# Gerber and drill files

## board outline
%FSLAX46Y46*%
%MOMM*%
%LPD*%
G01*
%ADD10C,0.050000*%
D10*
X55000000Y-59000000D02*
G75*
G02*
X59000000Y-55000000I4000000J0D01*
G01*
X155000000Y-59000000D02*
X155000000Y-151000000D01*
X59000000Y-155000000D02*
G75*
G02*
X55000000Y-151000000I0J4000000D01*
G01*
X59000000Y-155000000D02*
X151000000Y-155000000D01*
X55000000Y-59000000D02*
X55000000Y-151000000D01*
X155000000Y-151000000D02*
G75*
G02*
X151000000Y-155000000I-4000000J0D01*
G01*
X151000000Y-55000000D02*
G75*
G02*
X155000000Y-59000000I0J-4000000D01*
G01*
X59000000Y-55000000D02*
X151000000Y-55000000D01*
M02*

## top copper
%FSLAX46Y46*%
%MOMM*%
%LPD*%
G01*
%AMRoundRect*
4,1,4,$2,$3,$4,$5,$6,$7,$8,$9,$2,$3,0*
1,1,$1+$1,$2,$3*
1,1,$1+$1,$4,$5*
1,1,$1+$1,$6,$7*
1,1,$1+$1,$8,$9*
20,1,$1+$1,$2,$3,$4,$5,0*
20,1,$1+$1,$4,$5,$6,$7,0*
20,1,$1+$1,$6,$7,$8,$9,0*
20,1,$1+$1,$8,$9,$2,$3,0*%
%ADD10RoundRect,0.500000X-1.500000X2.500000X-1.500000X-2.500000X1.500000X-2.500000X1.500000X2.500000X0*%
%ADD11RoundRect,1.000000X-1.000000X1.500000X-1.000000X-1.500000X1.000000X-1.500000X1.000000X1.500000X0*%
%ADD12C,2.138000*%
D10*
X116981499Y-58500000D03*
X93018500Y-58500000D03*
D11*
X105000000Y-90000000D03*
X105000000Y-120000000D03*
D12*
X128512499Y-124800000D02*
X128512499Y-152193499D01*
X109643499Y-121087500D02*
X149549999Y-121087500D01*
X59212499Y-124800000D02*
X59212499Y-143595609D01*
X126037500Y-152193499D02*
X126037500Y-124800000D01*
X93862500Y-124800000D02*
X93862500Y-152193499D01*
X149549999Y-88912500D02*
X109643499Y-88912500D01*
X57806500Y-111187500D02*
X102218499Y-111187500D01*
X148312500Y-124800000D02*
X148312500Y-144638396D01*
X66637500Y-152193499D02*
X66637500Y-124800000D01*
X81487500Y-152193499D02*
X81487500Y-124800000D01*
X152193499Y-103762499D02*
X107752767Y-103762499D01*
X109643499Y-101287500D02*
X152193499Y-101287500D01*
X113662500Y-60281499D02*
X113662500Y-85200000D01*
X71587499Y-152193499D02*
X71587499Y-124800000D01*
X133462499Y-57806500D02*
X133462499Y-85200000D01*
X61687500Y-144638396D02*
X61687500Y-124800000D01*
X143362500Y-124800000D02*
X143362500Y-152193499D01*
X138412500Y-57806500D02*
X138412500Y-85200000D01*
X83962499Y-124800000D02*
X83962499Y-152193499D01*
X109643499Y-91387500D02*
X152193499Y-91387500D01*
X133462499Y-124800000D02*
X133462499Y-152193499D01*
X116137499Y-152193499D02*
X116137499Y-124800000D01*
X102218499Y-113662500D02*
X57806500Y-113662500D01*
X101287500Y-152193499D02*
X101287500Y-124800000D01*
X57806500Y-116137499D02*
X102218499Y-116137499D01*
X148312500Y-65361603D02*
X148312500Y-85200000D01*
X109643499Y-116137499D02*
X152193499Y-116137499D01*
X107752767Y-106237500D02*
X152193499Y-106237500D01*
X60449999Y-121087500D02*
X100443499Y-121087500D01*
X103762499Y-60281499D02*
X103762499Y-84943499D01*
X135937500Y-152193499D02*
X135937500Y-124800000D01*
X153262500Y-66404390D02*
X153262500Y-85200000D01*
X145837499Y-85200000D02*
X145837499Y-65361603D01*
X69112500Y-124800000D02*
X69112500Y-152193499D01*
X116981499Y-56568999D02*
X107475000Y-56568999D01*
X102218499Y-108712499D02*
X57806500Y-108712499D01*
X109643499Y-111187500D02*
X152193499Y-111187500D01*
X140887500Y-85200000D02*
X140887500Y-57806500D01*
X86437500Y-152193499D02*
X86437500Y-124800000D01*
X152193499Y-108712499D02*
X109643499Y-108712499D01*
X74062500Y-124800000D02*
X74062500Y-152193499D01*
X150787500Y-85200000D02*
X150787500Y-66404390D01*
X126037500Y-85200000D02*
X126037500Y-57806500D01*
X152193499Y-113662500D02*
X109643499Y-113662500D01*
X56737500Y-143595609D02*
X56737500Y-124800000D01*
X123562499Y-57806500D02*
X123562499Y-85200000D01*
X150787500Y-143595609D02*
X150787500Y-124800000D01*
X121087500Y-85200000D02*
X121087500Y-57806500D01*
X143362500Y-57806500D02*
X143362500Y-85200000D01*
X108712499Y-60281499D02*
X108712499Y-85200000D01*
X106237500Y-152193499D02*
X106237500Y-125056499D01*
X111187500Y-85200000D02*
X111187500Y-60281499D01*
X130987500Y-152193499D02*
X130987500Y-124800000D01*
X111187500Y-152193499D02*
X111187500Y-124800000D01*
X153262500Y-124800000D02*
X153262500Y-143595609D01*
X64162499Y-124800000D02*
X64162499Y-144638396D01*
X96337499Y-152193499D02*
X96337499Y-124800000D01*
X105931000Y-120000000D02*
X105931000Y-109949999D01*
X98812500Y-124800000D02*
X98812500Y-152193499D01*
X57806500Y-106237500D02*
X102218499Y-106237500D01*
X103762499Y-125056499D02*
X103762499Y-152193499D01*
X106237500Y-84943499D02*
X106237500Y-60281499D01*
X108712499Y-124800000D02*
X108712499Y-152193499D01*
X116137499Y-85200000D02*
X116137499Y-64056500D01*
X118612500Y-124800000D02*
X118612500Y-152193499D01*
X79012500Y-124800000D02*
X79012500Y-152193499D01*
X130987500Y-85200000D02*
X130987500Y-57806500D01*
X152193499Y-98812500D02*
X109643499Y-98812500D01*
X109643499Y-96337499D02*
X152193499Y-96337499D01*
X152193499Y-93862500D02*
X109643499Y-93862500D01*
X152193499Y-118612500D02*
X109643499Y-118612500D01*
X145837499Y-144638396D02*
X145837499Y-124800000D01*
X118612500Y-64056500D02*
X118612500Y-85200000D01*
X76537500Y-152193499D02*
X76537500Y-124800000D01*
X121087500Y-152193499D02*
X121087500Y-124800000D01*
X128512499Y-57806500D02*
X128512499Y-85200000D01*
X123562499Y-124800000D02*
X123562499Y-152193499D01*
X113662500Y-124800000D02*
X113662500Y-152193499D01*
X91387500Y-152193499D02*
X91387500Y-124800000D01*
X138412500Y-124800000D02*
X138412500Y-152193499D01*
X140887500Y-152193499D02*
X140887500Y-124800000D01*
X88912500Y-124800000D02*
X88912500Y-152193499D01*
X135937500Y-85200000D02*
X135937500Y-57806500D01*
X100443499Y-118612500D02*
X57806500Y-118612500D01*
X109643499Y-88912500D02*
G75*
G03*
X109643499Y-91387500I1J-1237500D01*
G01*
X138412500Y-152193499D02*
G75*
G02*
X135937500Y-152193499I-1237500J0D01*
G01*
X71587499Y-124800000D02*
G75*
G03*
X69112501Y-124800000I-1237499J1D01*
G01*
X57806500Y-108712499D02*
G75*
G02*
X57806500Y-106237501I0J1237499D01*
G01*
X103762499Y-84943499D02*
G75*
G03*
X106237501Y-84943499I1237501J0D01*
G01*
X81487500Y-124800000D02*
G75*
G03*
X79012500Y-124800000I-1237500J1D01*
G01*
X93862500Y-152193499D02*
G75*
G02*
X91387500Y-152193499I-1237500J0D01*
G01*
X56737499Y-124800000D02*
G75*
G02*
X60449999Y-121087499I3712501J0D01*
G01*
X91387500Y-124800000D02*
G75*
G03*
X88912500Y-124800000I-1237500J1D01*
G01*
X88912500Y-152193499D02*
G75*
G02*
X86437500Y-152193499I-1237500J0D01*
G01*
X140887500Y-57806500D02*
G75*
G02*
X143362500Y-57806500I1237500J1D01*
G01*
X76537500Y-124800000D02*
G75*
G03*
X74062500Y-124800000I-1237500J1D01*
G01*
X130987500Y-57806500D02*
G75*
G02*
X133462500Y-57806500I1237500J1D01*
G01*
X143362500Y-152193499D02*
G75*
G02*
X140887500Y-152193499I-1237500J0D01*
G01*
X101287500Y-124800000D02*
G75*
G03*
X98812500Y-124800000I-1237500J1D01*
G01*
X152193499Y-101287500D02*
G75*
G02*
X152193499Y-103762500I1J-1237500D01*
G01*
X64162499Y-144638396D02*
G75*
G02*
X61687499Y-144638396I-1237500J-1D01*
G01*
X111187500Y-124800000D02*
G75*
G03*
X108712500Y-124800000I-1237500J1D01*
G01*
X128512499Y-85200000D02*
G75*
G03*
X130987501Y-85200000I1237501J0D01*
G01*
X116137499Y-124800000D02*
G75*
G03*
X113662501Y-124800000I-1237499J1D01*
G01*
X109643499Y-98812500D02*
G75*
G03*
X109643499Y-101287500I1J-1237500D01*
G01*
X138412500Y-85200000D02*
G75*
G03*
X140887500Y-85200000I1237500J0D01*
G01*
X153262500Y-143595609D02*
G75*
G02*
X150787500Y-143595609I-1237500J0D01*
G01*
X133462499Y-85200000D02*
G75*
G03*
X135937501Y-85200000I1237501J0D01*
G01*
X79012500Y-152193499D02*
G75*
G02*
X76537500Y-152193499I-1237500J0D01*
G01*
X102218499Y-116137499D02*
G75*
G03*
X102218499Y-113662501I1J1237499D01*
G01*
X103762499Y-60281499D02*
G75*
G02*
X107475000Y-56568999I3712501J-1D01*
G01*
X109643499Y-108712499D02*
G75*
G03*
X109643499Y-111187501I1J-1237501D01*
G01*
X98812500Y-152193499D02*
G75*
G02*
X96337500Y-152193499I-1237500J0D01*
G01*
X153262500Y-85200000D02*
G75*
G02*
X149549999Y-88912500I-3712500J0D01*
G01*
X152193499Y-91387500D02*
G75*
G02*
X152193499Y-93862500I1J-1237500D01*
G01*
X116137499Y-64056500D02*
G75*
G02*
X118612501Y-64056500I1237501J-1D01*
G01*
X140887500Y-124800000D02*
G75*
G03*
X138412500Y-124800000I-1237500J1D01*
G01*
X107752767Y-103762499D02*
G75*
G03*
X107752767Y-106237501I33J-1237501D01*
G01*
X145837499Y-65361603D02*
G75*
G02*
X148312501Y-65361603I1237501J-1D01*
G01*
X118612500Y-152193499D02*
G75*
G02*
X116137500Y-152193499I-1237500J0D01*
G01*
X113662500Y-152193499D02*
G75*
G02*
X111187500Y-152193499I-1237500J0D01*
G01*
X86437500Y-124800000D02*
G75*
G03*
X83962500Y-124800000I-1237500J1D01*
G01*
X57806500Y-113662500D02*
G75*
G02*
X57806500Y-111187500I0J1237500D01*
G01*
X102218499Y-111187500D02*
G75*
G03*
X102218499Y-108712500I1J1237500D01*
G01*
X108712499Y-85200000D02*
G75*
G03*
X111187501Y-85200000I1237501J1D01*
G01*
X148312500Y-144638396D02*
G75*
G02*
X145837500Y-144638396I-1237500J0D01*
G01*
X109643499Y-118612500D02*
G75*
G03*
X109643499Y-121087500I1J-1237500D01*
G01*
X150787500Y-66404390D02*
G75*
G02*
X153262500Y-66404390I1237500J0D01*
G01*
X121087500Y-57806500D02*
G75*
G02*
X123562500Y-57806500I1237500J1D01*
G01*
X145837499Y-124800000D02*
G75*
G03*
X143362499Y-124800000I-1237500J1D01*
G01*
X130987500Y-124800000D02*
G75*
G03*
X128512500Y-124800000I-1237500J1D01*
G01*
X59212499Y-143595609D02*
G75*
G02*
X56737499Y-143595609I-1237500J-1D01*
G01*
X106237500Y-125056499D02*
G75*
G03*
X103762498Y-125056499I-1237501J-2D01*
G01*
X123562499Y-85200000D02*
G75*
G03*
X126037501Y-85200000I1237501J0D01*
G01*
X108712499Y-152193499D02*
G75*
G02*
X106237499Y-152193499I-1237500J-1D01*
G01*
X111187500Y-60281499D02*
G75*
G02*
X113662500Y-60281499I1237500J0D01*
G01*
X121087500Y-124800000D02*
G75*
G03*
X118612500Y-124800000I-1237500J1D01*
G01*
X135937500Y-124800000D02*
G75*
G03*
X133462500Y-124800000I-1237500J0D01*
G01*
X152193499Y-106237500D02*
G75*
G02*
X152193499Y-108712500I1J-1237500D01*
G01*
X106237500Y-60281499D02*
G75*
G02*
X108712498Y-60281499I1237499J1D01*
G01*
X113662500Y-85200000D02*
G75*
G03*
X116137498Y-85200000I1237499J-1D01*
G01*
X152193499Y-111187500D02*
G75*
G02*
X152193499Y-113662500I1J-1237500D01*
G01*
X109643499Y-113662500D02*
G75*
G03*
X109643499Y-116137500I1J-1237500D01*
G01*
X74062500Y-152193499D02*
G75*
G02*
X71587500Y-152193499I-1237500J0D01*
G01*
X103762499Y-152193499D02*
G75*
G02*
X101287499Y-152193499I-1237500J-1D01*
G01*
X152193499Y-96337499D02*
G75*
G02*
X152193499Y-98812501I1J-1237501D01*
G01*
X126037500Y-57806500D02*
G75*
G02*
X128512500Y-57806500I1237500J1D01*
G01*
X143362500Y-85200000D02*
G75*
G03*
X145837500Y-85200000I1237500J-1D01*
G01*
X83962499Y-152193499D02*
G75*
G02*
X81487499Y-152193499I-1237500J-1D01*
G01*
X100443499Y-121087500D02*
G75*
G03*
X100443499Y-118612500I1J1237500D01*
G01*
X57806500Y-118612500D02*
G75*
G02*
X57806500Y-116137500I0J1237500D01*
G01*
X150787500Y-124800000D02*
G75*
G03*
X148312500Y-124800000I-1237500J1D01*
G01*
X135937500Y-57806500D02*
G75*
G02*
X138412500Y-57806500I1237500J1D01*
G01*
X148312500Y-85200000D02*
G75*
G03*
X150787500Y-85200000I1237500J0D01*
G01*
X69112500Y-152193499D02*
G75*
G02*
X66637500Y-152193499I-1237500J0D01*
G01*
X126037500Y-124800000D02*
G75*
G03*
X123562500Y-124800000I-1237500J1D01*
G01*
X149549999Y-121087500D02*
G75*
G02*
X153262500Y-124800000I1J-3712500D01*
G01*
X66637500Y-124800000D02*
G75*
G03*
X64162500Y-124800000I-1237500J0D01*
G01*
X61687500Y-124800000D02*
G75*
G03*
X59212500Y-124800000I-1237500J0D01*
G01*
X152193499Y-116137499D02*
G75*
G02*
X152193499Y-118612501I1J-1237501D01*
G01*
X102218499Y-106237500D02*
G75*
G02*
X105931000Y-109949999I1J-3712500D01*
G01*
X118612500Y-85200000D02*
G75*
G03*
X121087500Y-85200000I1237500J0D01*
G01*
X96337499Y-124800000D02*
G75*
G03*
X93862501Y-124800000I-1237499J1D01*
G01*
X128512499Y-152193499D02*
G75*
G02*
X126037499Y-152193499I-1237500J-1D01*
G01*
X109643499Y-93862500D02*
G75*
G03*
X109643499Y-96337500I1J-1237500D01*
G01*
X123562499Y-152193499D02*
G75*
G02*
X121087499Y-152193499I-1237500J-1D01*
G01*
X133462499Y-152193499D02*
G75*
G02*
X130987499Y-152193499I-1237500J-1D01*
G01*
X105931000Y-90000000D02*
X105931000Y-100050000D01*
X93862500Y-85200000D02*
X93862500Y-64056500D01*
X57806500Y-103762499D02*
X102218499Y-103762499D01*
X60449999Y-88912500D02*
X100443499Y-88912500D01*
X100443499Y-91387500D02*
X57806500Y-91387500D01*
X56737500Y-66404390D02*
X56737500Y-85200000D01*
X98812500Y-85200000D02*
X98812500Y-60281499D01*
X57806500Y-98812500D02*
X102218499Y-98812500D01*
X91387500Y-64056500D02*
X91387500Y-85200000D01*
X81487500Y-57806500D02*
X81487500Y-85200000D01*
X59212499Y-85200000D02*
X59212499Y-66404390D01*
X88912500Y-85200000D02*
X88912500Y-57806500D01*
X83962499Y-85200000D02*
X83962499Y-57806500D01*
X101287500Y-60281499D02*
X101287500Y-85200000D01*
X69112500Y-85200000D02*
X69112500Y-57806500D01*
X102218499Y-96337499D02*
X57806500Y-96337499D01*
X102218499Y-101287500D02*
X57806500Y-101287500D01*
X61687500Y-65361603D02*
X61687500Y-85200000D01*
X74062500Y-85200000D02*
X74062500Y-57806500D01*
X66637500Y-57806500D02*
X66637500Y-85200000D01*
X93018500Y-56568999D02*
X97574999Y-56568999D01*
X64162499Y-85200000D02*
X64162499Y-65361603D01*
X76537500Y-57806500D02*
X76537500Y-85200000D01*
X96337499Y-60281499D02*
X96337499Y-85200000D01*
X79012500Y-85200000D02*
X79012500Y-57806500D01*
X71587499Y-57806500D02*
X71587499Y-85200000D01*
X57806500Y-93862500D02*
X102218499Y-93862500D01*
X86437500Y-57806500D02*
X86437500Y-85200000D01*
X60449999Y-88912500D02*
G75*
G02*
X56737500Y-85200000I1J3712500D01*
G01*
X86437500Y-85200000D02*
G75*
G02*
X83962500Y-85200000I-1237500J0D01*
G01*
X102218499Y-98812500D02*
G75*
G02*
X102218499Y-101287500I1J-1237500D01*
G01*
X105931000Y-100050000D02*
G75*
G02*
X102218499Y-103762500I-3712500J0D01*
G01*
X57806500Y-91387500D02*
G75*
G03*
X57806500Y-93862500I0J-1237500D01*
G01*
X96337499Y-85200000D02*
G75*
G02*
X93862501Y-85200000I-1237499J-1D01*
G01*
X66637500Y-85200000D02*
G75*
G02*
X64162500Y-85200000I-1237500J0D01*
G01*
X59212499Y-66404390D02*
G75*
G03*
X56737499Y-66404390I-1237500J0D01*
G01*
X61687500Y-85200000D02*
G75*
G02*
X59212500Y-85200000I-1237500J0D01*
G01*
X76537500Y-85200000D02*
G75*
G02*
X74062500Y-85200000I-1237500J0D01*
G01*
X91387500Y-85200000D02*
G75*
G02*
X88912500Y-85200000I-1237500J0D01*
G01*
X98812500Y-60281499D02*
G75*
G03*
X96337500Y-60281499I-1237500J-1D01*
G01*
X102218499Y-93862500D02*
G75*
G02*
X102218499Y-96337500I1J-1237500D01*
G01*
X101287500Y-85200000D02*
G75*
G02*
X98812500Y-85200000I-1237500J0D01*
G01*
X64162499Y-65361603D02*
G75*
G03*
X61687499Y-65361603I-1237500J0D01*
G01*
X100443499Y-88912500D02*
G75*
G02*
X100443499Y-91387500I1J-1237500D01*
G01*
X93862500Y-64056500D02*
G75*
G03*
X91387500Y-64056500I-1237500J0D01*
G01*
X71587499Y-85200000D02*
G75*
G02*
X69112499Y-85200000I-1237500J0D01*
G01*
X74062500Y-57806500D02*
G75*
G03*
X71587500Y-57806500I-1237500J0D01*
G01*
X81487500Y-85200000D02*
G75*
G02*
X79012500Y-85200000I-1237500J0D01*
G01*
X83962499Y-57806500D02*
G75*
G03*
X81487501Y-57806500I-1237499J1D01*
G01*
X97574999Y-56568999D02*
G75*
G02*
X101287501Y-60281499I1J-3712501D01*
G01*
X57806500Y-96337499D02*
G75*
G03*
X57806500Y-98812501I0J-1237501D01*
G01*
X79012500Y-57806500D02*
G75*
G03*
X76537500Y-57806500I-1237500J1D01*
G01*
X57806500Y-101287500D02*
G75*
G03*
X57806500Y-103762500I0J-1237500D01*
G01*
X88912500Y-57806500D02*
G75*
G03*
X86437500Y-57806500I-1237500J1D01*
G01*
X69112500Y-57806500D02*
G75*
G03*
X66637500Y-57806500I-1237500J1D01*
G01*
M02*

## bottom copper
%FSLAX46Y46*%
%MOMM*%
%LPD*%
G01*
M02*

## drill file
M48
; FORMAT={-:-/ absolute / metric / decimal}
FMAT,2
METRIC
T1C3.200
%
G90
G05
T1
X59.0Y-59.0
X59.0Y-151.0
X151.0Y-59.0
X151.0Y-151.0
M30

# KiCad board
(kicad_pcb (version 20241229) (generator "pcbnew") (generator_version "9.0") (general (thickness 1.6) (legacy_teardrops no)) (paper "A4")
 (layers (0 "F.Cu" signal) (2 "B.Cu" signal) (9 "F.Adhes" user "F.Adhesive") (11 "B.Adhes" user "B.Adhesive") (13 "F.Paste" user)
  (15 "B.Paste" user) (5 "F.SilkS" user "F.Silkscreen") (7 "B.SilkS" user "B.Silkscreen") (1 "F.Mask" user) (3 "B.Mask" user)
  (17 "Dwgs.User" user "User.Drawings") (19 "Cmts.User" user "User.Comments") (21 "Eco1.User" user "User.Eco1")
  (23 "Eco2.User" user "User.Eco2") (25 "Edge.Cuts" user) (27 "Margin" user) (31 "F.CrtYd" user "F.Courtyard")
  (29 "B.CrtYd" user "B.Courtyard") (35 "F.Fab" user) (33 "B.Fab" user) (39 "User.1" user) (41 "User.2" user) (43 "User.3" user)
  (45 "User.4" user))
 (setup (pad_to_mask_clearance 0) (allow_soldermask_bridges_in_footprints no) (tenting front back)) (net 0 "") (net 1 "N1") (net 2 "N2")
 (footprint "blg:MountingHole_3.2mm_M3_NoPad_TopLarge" (layer "F.Cu") (at 151 59)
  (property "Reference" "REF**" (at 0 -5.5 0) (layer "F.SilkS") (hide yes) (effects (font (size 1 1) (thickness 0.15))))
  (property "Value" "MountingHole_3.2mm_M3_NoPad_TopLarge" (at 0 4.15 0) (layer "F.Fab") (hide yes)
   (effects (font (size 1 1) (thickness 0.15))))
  (pad "" np_thru_hole circle (at 0 0) (size 7.6 7.6) (drill 3.2) (layers) (zone_connect 2)))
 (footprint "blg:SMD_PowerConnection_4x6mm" (layer "F.Cu") (at 116.981499 58.5 -90)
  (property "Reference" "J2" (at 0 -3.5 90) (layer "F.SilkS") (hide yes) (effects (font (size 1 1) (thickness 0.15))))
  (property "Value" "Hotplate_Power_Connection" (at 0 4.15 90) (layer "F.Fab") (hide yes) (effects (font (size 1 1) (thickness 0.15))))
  (pad "1" smd roundrect (at 0 0 270) (size 6 4) (layers "F.Cu" "F.Mask" "F.Paste") (roundrect_rratio 0.125) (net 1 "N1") (zone_connect 2)))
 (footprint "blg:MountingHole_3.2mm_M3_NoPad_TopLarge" (layer "F.Cu") (at 59 151)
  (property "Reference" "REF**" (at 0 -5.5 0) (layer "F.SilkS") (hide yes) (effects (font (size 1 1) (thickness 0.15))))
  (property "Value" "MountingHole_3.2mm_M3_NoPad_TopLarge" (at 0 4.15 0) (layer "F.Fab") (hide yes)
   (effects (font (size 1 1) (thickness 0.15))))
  (pad "" np_thru_hole circle (at 0 0) (size 7.6 7.6) (drill 3.2) (layers) (zone_connect 2)))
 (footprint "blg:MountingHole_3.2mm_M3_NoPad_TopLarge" (layer "F.Cu") (at 151 151)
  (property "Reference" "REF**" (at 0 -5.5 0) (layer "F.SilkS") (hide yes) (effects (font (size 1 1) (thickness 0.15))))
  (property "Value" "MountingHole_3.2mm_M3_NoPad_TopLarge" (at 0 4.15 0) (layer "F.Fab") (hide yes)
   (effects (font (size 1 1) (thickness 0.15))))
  (pad "" np_thru_hole circle (at 0 0) (size 7.6 7.6) (drill 3.2) (layers) (zone_connect 2)))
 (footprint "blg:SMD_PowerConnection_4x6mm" (layer "F.Cu") (at 93.0185 58.5 -90)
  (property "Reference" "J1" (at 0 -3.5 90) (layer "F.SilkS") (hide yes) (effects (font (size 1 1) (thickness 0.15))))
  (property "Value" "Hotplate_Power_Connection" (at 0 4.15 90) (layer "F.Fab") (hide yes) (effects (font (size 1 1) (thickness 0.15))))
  (pad "1" smd roundrect (at 0 0 270) (size 6 4) (layers "F.Cu" "F.Mask" "F.Paste") (roundrect_rratio 0.125) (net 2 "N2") (zone_connect 2)))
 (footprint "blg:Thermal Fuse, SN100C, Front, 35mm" (layer "F.Cu") (at 105 105 -90)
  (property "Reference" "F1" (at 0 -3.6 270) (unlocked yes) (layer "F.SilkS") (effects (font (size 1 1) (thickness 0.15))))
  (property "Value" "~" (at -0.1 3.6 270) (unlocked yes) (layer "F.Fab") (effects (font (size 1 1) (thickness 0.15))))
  (pad "1" smd roundrect (at -15 0 270) (size 5 4) (layers "F.Cu" "F.Mask") (roundrect_rratio 0.25) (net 2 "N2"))
  (pad "2" smd roundrect (at 15 0 270) (size 5 4) (layers "F.Cu" "F.Mask") (roundrect_rratio 0.25) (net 1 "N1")))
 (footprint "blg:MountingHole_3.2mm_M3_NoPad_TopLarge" (layer "F.Cu") (at 59 59)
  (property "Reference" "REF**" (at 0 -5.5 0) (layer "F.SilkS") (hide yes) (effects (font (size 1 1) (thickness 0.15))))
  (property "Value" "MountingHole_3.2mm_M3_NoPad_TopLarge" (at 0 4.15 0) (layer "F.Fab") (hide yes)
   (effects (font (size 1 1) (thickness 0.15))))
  (pad "" np_thru_hole circle (at 0 0) (size 7.6 7.6) (drill 3.2) (layers) (zone_connect 2)))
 (gr_arc (start 55 59) (mid 56.171573 56.171573) (end 59 55) (stroke (width 0.05) (type solid)) (layer "Edge.Cuts"))
 (gr_line (start 155 59) (end 155 151) (stroke (width 0.05) (type default)) (layer "Edge.Cuts"))
 (gr_arc (start 59 155) (mid 56.171573 153.828427) (end 55 151) (stroke (width 0.05) (type solid)) (layer "Edge.Cuts"))
 (gr_line (start 59 155) (end 151 155) (stroke (width 0.05) (type default)) (layer "Edge.Cuts"))
 (gr_line (start 55 59) (end 55 151) (stroke (width 0.05) (type default)) (layer "Edge.Cuts"))
 (gr_arc (start 155 151) (mid 153.828427 153.828427) (end 151 155) (stroke (width 0.05) (type solid)) (layer "Edge.Cuts"))
 (gr_arc (start 151 55) (mid 153.828427 56.171573) (end 155 59) (stroke (width 0.05) (type solid)) (layer "Edge.Cuts"))
 (gr_line (start 59 55) (end 151 55) (stroke (width 0.05) (type default)) (layer "Edge.Cuts"))
 (segment (start 128.512499 124.8) (end 128.512499 152.193499) (width 2.138) (layer "F.Cu") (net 1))
 (segment (start 109.643499 121.0875) (end 149.549999 121.0875) (width 2.138) (layer "F.Cu") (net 1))
 (segment (start 59.212499 124.8) (end 59.212499 143.595609) (width 2.138) (layer "F.Cu") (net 1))
 (segment (start 126.0375 152.193499) (end 126.0375 124.8) (width 2.138) (layer "F.Cu") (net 1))
 (segment (start 93.8625 124.8) (end 93.8625 152.193499) (width 2.138) (layer "F.Cu") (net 1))
 (segment (start 149.549999 88.9125) (end 109.643499 88.9125) (width 2.138) (layer "F.Cu") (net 1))
 (segment (start 57.8065 111.1875) (end 102.218499 111.1875) (width 2.138) (layer "F.Cu") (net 1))
 (segment (start 148.3125 124.8) (end 148.3125 144.638396) (width 2.138) (layer "F.Cu") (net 1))
 (segment (start 66.6375 152.193499) (end 66.6375 124.8) (width 2.138) (layer "F.Cu") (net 1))
 (segment (start 81.4875 152.193499) (end 81.4875 124.8) (width 2.138) (layer "F.Cu") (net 1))
 (segment (start 152.193499 103.762499) (end 107.752767 103.762499) (width 2.138) (layer "F.Cu") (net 1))
 (segment (start 109.643499 101.2875) (end 152.193499 101.2875) (width 2.138) (layer "F.Cu") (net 1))
 (segment (start 113.6625 60.281499) (end 113.6625 85.2) (width 2.138) (layer "F.Cu") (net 1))
 (segment (start 71.587499 152.193499) (end 71.587499 124.8) (width 2.138) (layer "F.Cu") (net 1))
 (segment (start 133.462499 57.8065) (end 133.462499 85.2) (width 2.138) (layer "F.Cu") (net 1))
 (segment (start 61.6875 144.638396) (end 61.6875 124.8) (width 2.138) (layer "F.Cu") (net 1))
 (segment (start 143.3625 124.8) (end 143.3625 152.193499) (width 2.138) (layer "F.Cu") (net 1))
 (segment (start 138.4125 57.8065) (end 138.4125 85.2) (width 2.138) (layer "F.Cu") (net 1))
 (segment (start 83.962499 124.8) (end 83.962499 152.193499) (width 2.138) (layer "F.Cu") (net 1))
 (segment (start 109.643499 91.3875) (end 152.193499 91.3875) (width 2.138) (layer "F.Cu") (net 1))
 (segment (start 133.462499 124.8) (end 133.462499 152.193499) (width 2.138) (layer "F.Cu") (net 1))
 (segment (start 116.137499 152.193499) (end 116.137499 124.8) (width 2.138) (layer "F.Cu") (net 1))
 (segment (start 102.218499 113.6625) (end 57.8065 113.6625) (width 2.138) (layer "F.Cu") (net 1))
 (segment (start 101.2875 152.193499) (end 101.2875 124.8) (width 2.138) (layer "F.Cu") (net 1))
 (segment (start 57.8065 116.137499) (end 102.218499 116.137499) (width 2.138) (layer "F.Cu") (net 1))
 (segment (start 148.3125 65.361603) (end 148.3125 85.2) (width 2.138) (layer "F.Cu") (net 1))
 (segment (start 109.643499 116.137499) (end 152.193499 116.137499) (width 2.138) (layer "F.Cu") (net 1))
 (segment (start 107.752767 106.2375) (end 152.193499 106.2375) (width 2.138) (layer "F.Cu") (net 1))
 (segment (start 60.449999 121.0875) (end 100.443499 121.0875) (width 2.138) (layer "F.Cu") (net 1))
 (segment (start 103.762499 60.281499) (end 103.762499 84.943499) (width 2.138) (layer "F.Cu") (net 1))
 (segment (start 135.9375 152.193499) (end 135.9375 124.8) (width 2.138) (layer "F.Cu") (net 1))
 (segment (start 153.2625 66.40439) (end 153.2625 85.2) (width 2.138) (layer "F.Cu") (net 1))
 (segment (start 145.837499 85.2) (end 145.837499 65.361603) (width 2.138) (layer "F.Cu") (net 1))
 (segment (start 69.1125 124.8) (end 69.1125 152.193499) (width 2.138) (layer "F.Cu") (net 1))
 (segment (start 116.981499 56.568999) (end 107.475 56.568999) (width 2.138) (layer "F.Cu") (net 1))
 (segment (start 102.218499 108.712499) (end 57.8065 108.712499) (width 2.138) (layer "F.Cu") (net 1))
 (segment (start 109.643499 111.1875) (end 152.193499 111.1875) (width 2.138) (layer "F.Cu") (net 1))
 (segment (start 140.8875 85.2) (end 140.8875 57.8065) (width 2.138) (layer "F.Cu") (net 1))
 (segment (start 86.4375 152.193499) (end 86.4375 124.8) (width 2.138) (layer "F.Cu") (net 1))
 (segment (start 152.193499 108.712499) (end 109.643499 108.712499) (width 2.138) (layer "F.Cu") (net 1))
 (segment (start 74.0625 124.8) (end 74.0625 152.193499) (width 2.138) (layer "F.Cu") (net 1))
 (segment (start 150.7875 85.2) (end 150.7875 66.40439) (width 2.138) (layer "F.Cu") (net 1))
 (segment (start 126.0375 85.2) (end 126.0375 57.8065) (width 2.138) (layer "F.Cu") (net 1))
 (segment (start 152.193499 113.6625) (end 109.643499 113.6625) (width 2.138) (layer "F.Cu") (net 1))
 (segment (start 56.7375 143.595609) (end 56.7375 124.8) (width 2.138) (layer "F.Cu") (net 1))
 (segment (start 123.562499 57.8065) (end 123.562499 85.2) (width 2.138) (layer "F.Cu") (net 1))
 (segment (start 150.7875 143.595609) (end 150.7875 124.8) (width 2.138) (layer "F.Cu") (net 1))
 (segment (start 121.0875 85.2) (end 121.0875 57.8065) (width 2.138) (layer "F.Cu") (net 1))
 (segment (start 143.3625 57.8065) (end 143.3625 85.2) (width 2.138) (layer "F.Cu") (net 1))
 (segment (start 108.712499 60.281499) (end 108.712499 85.2) (width 2.138) (layer "F.Cu") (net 1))
 (segment (start 106.2375 152.193499) (end 106.2375 125.056499) (width 2.138) (layer "F.Cu") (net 1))
 (segment (start 111.1875 85.2) (end 111.1875 60.281499) (width 2.138) (layer "F.Cu") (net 1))
 (segment (start 130.9875 152.193499) (end 130.9875 124.8) (width 2.138) (layer "F.Cu") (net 1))
 (segment (start 111.1875 152.193499) (end 111.1875 124.8) (width 2.138) (layer "F.Cu") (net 1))
 (segment (start 153.2625 124.8) (end 153.2625 143.595609) (width 2.138) (layer "F.Cu") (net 1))
 (segment (start 64.162499 124.8) (end 64.162499 144.638396) (width 2.138) (layer "F.Cu") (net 1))
 (segment (start 96.337499 152.193499) (end 96.337499 124.8) (width 2.138) (layer "F.Cu") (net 1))
 (segment (start 105.931 120) (end 105.931 109.949999) (width 2.138) (layer "F.Cu") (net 1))
 (segment (start 98.8125 124.8) (end 98.8125 152.193499) (width 2.138) (layer "F.Cu") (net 1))
 (segment (start 57.8065 106.2375) (end 102.218499 106.2375) (width 2.138) (layer "F.Cu") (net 1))
 (segment (start 103.762499 125.056499) (end 103.762499 152.193499) (width 2.138) (layer "F.Cu") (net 1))
 (segment (start 106.2375 84.943499) (end 106.2375 60.281499) (width 2.138) (layer "F.Cu") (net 1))
 (segment (start 108.712499 124.8) (end 108.712499 152.193499) (width 2.138) (layer "F.Cu") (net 1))
 (segment (start 116.137499 85.2) (end 116.137499 64.0565) (width 2.138) (layer "F.Cu") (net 1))
 (segment (start 118.6125 124.8) (end 118.6125 152.193499) (width 2.138) (layer "F.Cu") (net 1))
 (segment (start 79.0125 124.8) (end 79.0125 152.193499) (width 2.138) (layer "F.Cu") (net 1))
 (segment (start 130.9875 85.2) (end 130.9875 57.8065) (width 2.138) (layer "F.Cu") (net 1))
 (segment (start 152.193499 98.8125) (end 109.643499 98.8125) (width 2.138) (layer "F.Cu") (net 1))
 (segment (start 109.643499 96.337499) (end 152.193499 96.337499) (width 2.138) (layer "F.Cu") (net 1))
 (segment (start 152.193499 93.8625) (end 109.643499 93.8625) (width 2.138) (layer "F.Cu") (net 1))
 (segment (start 152.193499 118.6125) (end 109.643499 118.6125) (width 2.138) (layer "F.Cu") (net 1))
 (segment (start 145.837499 144.638396) (end 145.837499 124.8) (width 2.138) (layer "F.Cu") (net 1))
 (segment (start 118.6125 64.0565) (end 118.6125 85.2) (width 2.138) (layer "F.Cu") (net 1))
 (segment (start 76.5375 152.193499) (end 76.5375 124.8) (width 2.138) (layer "F.Cu") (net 1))
 (segment (start 121.0875 152.193499) (end 121.0875 124.8) (width 2.138) (layer "F.Cu") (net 1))
 (segment (start 128.512499 57.8065) (end 128.512499 85.2) (width 2.138) (layer "F.Cu") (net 1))
 (segment (start 123.562499 124.8) (end 123.562499 152.193499) (width 2.138) (layer "F.Cu") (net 1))
 (segment (start 113.6625 124.8) (end 113.6625 152.193499) (width 2.138) (layer "F.Cu") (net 1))
 (segment (start 91.3875 152.193499) (end 91.3875 124.8) (width 2.138) (layer "F.Cu") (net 1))
 (segment (start 138.4125 124.8) (end 138.4125 152.193499) (width 2.138) (layer "F.Cu") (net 1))
 (segment (start 140.8875 152.193499) (end 140.8875 124.8) (width 2.138) (layer "F.Cu") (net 1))
 (segment (start 88.9125 124.8) (end 88.9125 152.193499) (width 2.138) (layer "F.Cu") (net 1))
 (segment (start 135.9375 85.2) (end 135.9375 57.8065) (width 2.138) (layer "F.Cu") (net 1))
 (segment (start 100.443499 118.6125) (end 57.8065 118.6125) (width 2.138) (layer "F.Cu") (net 1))
 (arc (start 109.643499 88.9125) (mid 108.405999 90.149999) (end 109.643499 91.3875) (width 2.138) (layer "F.Cu") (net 1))
 (arc (start 138.4125 152.193499) (mid 137.174999 153.430999) (end 135.9375 152.193499) (width 2.138) (layer "F.Cu") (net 1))
 (arc (start 71.587499 124.8) (mid 70.35 123.562499) (end 69.1125 124.8) (width 2.138) (layer "F.Cu") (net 1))
 (arc (start 57.8065 108.712499) (mid 56.568999 107.475) (end 57.8065 106.2375) (width 2.138) (layer "F.Cu") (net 1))
 (arc (start 103.762499 84.943499) (mid 105 86.181) (end 106.2375 84.943499) (width 2.138) (layer "F.Cu") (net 1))
 (arc (start 81.4875 124.8) (mid 80.25 123.562499) (end 79.0125 124.8) (width 2.138) (layer "F.Cu") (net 1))
 (arc (start 93.8625 152.193499) (mid 92.625 153.430999) (end 91.3875 152.193499) (width 2.138) (layer "F.Cu") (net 1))
 (arc (start 56.737499 124.8) (mid 57.824866 122.174866) (end 60.449999 121.0875) (width 2.138) (layer "F.Cu") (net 1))
 (arc (start 91.3875 124.8) (mid 90.149999 123.562499) (end 88.9125 124.8) (width 2.138) (layer "F.Cu") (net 1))
 (arc (start 88.9125 152.193499) (mid 87.675 153.430999) (end 86.4375 152.193499) (width 2.138) (layer "F.Cu") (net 1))
 (arc (start 140.8875 57.8065) (mid 142.125 56.568999) (end 143.3625 57.8065) (width 2.138) (layer "F.Cu") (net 1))
 (arc (start 76.5375 124.8) (mid 75.3 123.562499) (end 74.0625 124.8) (width 2.138) (layer "F.Cu") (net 1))
 (arc (start 130.9875 57.8065) (mid 132.225 56.568999) (end 133.462499 57.8065) (width 2.138) (layer "F.Cu") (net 1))
 (arc (start 143.3625 152.193499) (mid 142.125 153.430999) (end 140.8875 152.193499) (width 2.138) (layer "F.Cu") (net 1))
 (arc (start 101.2875 124.8) (mid 100.05 123.562499) (end 98.8125 124.8) (width 2.138) (layer "F.Cu") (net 1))
 (arc (start 152.193499 101.2875) (mid 153.430999 102.524999) (end 152.193499 103.762499) (width 2.138) (layer "F.Cu") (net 1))
 (arc (start 64.162499 144.638396) (mid 62.925 145.875896) (end 61.6875 144.638396) (width 2.138) (layer "F.Cu") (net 1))
 (arc (start 111.1875 124.8) (mid 109.949999 123.562499) (end 108.712499 124.8) (width 2.138) (layer "F.Cu") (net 1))
 (arc (start 128.512499 85.2) (mid 129.75 86.4375) (end 130.9875 85.2) (width 2.138) (layer "F.Cu") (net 1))
 (arc (start 116.137499 124.8) (mid 114.899999 123.562499) (end 113.6625 124.8) (width 2.138) (layer "F.Cu") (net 1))
 (arc (start 109.643499 98.8125) (mid 108.405999 100.05) (end 109.643499 101.2875) (width 2.138) (layer "F.Cu") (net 1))
 (arc (start 138.4125 85.2) (mid 139.65 86.4375) (end 140.8875 85.2) (width 2.138) (layer "F.Cu") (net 1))
 (arc (start 153.2625 143.595609) (mid 152.025 144.833109) (end 150.7875 143.595609) (width 2.138) (layer "F.Cu") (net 1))
 (arc (start 133.462499 85.2) (mid 134.7 86.4375) (end 135.9375 85.2) (width 2.138) (layer "F.Cu") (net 1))
 (arc (start 79.0125 152.193499) (mid 77.774999 153.430999) (end 76.5375 152.193499) (width 2.138) (layer "F.Cu") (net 1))
 (arc (start 102.218499 116.137499) (mid 103.455999 114.899999) (end 102.218499 113.6625) (width 2.138) (layer "F.Cu") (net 1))
 (arc (start 103.762499 60.281499) (mid 104.849866 57.656366) (end 107.475 56.568999) (width 2.138) (layer "F.Cu") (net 1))
 (arc (start 109.643499 108.712499) (mid 108.405999 109.949999) (end 109.643499 111.1875) (width 2.138) (layer "F.Cu") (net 1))
 (arc (start 98.8125 152.193499) (mid 97.574999 153.430999) (end 96.337499 152.193499) (width 2.138) (layer "F.Cu") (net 1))
 (arc (start 153.2625 85.2) (mid 152.175133 87.825133) (end 149.549999 88.9125) (width 2.138) (layer "F.Cu") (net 1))
 (arc (start 152.193499 91.3875) (mid 153.430999 92.625) (end 152.193499 93.8625) (width 2.138) (layer "F.Cu") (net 1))
 (arc (start 116.137499 64.0565) (mid 117.375 62.819) (end 118.6125 64.0565) (width 2.138) (layer "F.Cu") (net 1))
 (arc (start 140.8875 124.8) (mid 139.65 123.562499) (end 138.4125 124.8) (width 2.138) (layer "F.Cu") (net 1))
 (arc (start 107.752767 103.762499) (mid 106.515267 105) (end 107.752767 106.2375) (width 2.138) (layer "F.Cu") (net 1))
 (arc (start 145.837499 65.361603) (mid 147.075 64.124103) (end 148.3125 65.361603) (width 2.138) (layer "F.Cu") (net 1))
 (arc (start 118.6125 152.193499) (mid 117.375 153.430999) (end 116.137499 152.193499) (width 2.138) (layer "F.Cu") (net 1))
 (arc (start 113.6625 152.193499) (mid 112.425 153.430999) (end 111.1875 152.193499) (width 2.138) (layer "F.Cu") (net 1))
 (arc (start 86.4375 124.8) (mid 85.2 123.562499) (end 83.962499 124.8) (width 2.138) (layer "F.Cu") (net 1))
 (arc (start 57.8065 113.6625) (mid 56.568999 112.425) (end 57.8065 111.1875) (width 2.138) (layer "F.Cu") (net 1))
 (arc (start 102.218499 111.1875) (mid 103.455999 109.949999) (end 102.218499 108.712499) (width 2.138) (layer "F.Cu") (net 1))
 (arc (start 108.712499 85.2) (mid 109.949999 86.4375) (end 111.1875 85.2) (width 2.138) (layer "F.Cu") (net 1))
 (arc (start 148.3125 144.638396) (mid 147.075 145.875896) (end 145.837499 144.638396) (width 2.138) (layer "F.Cu") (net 1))
 (arc (start 109.643499 118.6125) (mid 108.405999 119.85) (end 109.643499 121.0875) (width 2.138) (layer "F.Cu") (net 1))
 (arc (start 150.7875 66.40439) (mid 152.025 65.16689) (end 153.2625 66.40439) (width 2.138) (layer "F.Cu") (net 1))
 (arc (start 121.0875 57.8065) (mid 122.324999 56.568999) (end 123.562499 57.8065) (width 2.138) (layer "F.Cu") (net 1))
 (arc (start 145.837499 124.8) (mid 144.6 123.562499) (end 143.3625 124.8) (width 2.138) (layer "F.Cu") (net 1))
 (arc (start 130.9875 124.8) (mid 129.75 123.562499) (end 128.512499 124.8) (width 2.138) (layer "F.Cu") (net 1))
 (arc (start 59.212499 143.595609) (mid 57.975 144.833109) (end 56.7375 143.595609) (width 2.138) (layer "F.Cu") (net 1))
 (arc (start 106.2375 125.056499) (mid 105 123.819) (end 103.762499 125.056499) (width 2.138) (layer "F.Cu") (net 1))
 (arc (start 123.562499 85.2) (mid 124.8 86.4375) (end 126.0375 85.2) (width 2.138) (layer "F.Cu") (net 1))
 (arc (start 108.712499 152.193499) (mid 107.475 153.430999) (end 106.2375 152.193499) (width 2.138) (layer "F.Cu") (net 1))
 (arc (start 111.1875 60.281499) (mid 112.425 59.043999) (end 113.6625 60.281499) (width 2.138) (layer "F.Cu") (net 1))
 (arc (start 121.0875 124.8) (mid 119.85 123.562499) (end 118.6125 124.8) (width 2.138) (layer "F.Cu") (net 1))
 (arc (start 135.9375 124.8) (mid 134.7 123.562499) (end 133.462499 124.8) (width 2.138) (layer "F.Cu") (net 1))
 (arc (start 152.193499 106.2375) (mid 153.430999 107.475) (end 152.193499 108.712499) (width 2.138) (layer "F.Cu") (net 1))
 (arc (start 106.2375 60.281499) (mid 107.475 59.043999) (end 108.712499 60.281499) (width 2.138) (layer "F.Cu") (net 1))
 (arc (start 113.6625 85.2) (mid 114.899999 86.4375) (end 116.137499 85.2) (width 2.138) (layer "F.Cu") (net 1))
 (arc (start 152.193499 111.1875) (mid 153.430999 112.425) (end 152.193499 113.6625) (width 2.138) (layer "F.Cu") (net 1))
 (arc (start 109.643499 113.6625) (mid 108.405999 114.899999) (end 109.643499 116.137499) (width 2.138) (layer "F.Cu") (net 1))
 (arc (start 74.0625 152.193499) (mid 72.825 153.430999) (end 71.587499 152.193499) (width 2.138) (layer "F.Cu") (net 1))
 (arc (start 103.762499 152.193499) (mid 102.524999 153.430999) (end 101.2875 152.193499) (width 2.138) (layer "F.Cu") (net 1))
 (arc (start 152.193499 96.337499) (mid 153.430999 97.574999) (end 152.193499 98.8125) (width 2.138) (layer "F.Cu") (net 1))
 (arc (start 126.0375 57.8065) (mid 127.275 56.568999) (end 128.512499 57.8065) (width 2.138) (layer "F.Cu") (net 1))
 (arc (start 143.3625 85.2) (mid 144.6 86.4375) (end 145.837499 85.2) (width 2.138) (layer "F.Cu") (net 1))
 (arc (start 83.962499 152.193499) (mid 82.725 153.430999) (end 81.4875 152.193499) (width 2.138) (layer "F.Cu") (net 1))
 (arc (start 100.443499 121.0875) (mid 101.681 119.85) (end 100.443499 118.6125) (width 2.138) (layer "F.Cu") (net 1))
 (arc (start 57.8065 118.6125) (mid 56.568999 117.375) (end 57.8065 116.137499) (width 2.138) (layer "F.Cu") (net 1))
 (arc (start 150.7875 124.8) (mid 149.549999 123.562499) (end 148.3125 124.8) (width 2.138) (layer "F.Cu") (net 1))
 (arc (start 135.9375 57.8065) (mid 137.174999 56.568999) (end 138.4125 57.8065) (width 2.138) (layer "F.Cu") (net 1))
 (arc (start 148.3125 85.2) (mid 149.549999 86.4375) (end 150.7875 85.2) (width 2.138) (layer "F.Cu") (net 1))
 (arc (start 69.1125 152.193499) (mid 67.874999 153.430999) (end 66.6375 152.193499) (width 2.138) (layer "F.Cu") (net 1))
 (arc (start 126.0375 124.8) (mid 124.8 123.562499) (end 123.562499 124.8) (width 2.138) (layer "F.Cu") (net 1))
 (arc (start 149.549999 121.0875) (mid 152.175133 122.174866) (end 153.2625 124.8) (width 2.138) (layer "F.Cu") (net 1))
 (arc (start 66.6375 124.8) (mid 65.4 123.562499) (end 64.162499 124.8) (width 2.138) (layer "F.Cu") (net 1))
 (arc (start 61.6875 124.8) (mid 60.449999 123.562499) (end 59.212499 124.8) (width 2.138) (layer "F.Cu") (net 1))
 (arc (start 152.193499 116.137499) (mid 153.430999 117.375) (end 152.193499 118.6125) (width 2.138) (layer "F.Cu") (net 1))
 (arc (start 102.218499 106.2375) (mid 104.843633 107.324866) (end 105.931 109.949999) (width 2.138) (layer "F.Cu") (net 1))
 (arc (start 118.6125 85.2) (mid 119.85 86.4375) (end 121.0875 85.2) (width 2.138) (layer "F.Cu") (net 1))
 (arc (start 96.337499 124.8) (mid 95.1 123.562499) (end 93.8625 124.8) (width 2.138) (layer "F.Cu") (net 1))
 (arc (start 128.512499 152.193499) (mid 127.275 153.430999) (end 126.0375 152.193499) (width 2.138) (layer "F.Cu") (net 1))
 (arc (start 109.643499 93.8625) (mid 108.405999 95.1) (end 109.643499 96.337499) (width 2.138) (layer "F.Cu") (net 1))
 (arc (start 123.562499 152.193499) (mid 122.324999 153.430999) (end 121.0875 152.193499) (width 2.138) (layer "F.Cu") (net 1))
 (arc (start 133.462499 152.193499) (mid 132.225 153.430999) (end 130.9875 152.193499) (width 2.138) (layer "F.Cu") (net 1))
 (segment (start 105.931 90) (end 105.931 100.05) (width 2.138) (layer "F.Cu") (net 2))
 (segment (start 93.8625 85.2) (end 93.8625 64.0565) (width 2.138) (layer "F.Cu") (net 2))
 (segment (start 57.8065 103.762499) (end 102.218499 103.762499) (width 2.138) (layer "F.Cu") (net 2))
 (segment (start 60.449999 88.9125) (end 100.443499 88.9125) (width 2.138) (layer "F.Cu") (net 2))
 (segment (start 100.443499 91.3875) (end 57.8065 91.3875) (width 2.138) (layer "F.Cu") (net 2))
 (segment (start 56.7375 66.40439) (end 56.7375 85.2) (width 2.138) (layer "F.Cu") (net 2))
 (segment (start 98.8125 85.2) (end 98.8125 60.281499) (width 2.138) (layer "F.Cu") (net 2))
 (segment (start 57.8065 98.8125) (end 102.218499 98.8125) (width 2.138) (layer "F.Cu") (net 2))
 (segment (start 91.3875 64.0565) (end 91.3875 85.2) (width 2.138) (layer "F.Cu") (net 2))
 (segment (start 81.4875 57.8065) (end 81.4875 85.2) (width 2.138) (layer "F.Cu") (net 2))
 (segment (start 59.212499 85.2) (end 59.212499 66.40439) (width 2.138) (layer "F.Cu") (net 2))
 (segment (start 88.9125 85.2) (end 88.9125 57.8065) (width 2.138) (layer "F.Cu") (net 2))
 (segment (start 83.962499 85.2) (end 83.962499 57.8065) (width 2.138) (layer "F.Cu") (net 2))
 (segment (start 101.2875 60.281499) (end 101.2875 85.2) (width 2.138) (layer "F.Cu") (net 2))
 (segment (start 69.1125 85.2) (end 69.1125 57.8065) (width 2.138) (layer "F.Cu") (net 2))
 (segment (start 102.218499 96.337499) (end 57.8065 96.337499) (width 2.138) (layer "F.Cu") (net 2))
 (segment (start 102.218499 101.2875) (end 57.8065 101.2875) (width 2.138) (layer "F.Cu") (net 2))
 (segment (start 61.6875 65.361603) (end 61.6875 85.2) (width 2.138) (layer "F.Cu") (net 2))
 (segment (start 74.0625 85.2) (end 74.0625 57.8065) (width 2.138) (layer "F.Cu") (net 2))
 (segment (start 66.6375 57.8065) (end 66.6375 85.2) (width 2.138) (layer "F.Cu") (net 2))
 (segment (start 93.0185 56.568999) (end 97.574999 56.568999) (width 2.138) (layer "F.Cu") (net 2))
 (segment (start 64.162499 85.2) (end 64.162499 65.361603) (width 2.138) (layer "F.Cu") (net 2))
 (segment (start 76.5375 57.8065) (end 76.5375 85.2) (width 2.138) (layer "F.Cu") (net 2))
 (segment (start 96.337499 60.281499) (end 96.337499 85.2) (width 2.138) (layer "F.Cu") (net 2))
 (segment (start 79.0125 85.2) (end 79.0125 57.8065) (width 2.138) (layer "F.Cu") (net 2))
 (segment (start 71.587499 57.8065) (end 71.587499 85.2) (width 2.138) (layer "F.Cu") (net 2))
 (segment (start 57.8065 93.8625) (end 102.218499 93.8625) (width 2.138) (layer "F.Cu") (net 2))
 (segment (start 86.4375 57.8065) (end 86.4375 85.2) (width 2.138) (layer "F.Cu") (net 2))
 (arc (start 60.449999 88.9125) (mid 57.824866 87.825133) (end 56.737499 85.2) (width 2.138) (layer "F.Cu") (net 2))
 (arc (start 86.4375 85.2) (mid 85.2 86.4375) (end 83.962499 85.2) (width 2.138) (layer "F.Cu") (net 2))
 (arc (start 102.218499 98.8125) (mid 103.455999 100.05) (end 102.218499 101.2875) (width 2.138) (layer "F.Cu") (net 2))
 (arc (start 105.931 100.05) (mid 104.843633 102.675133) (end 102.218499 103.762499) (width 2.138) (layer "F.Cu") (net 2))
 (arc (start 57.8065 91.3875) (mid 56.568999 92.625) (end 57.8065 93.8625) (width 2.138) (layer "F.Cu") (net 2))
 (arc (start 96.337499 85.2) (mid 95.1 86.4375) (end 93.8625 85.2) (width 2.138) (layer "F.Cu") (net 2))
 (arc (start 66.6375 85.2) (mid 65.4 86.4375) (end 64.162499 85.2) (width 2.138) (layer "F.Cu") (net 2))
 (arc (start 59.212499 66.40439) (mid 57.975 65.16689) (end 56.7375 66.40439) (width 2.138) (layer "F.Cu") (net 2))
 (arc (start 61.6875 85.2) (mid 60.449999 86.4375) (end 59.212499 85.2) (width 2.138) (layer "F.Cu") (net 2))
 (arc (start 76.5375 85.2) (mid 75.3 86.4375) (end 74.0625 85.2) (width 2.138) (layer "F.Cu") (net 2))
 (arc (start 91.3875 85.2) (mid 90.149999 86.4375) (end 88.9125 85.2) (width 2.138) (layer "F.Cu") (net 2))
 (arc (start 98.8125 60.281499) (mid 97.574999 59.043999) (end 96.337499 60.281499) (width 2.138) (layer "F.Cu") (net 2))
 (arc (start 102.218499 93.8625) (mid 103.455999 95.1) (end 102.218499 96.337499) (width 2.138) (layer "F.Cu") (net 2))
 (arc (start 101.2875 85.2) (mid 100.05 86.4375) (end 98.8125 85.2) (width 2.138) (layer "F.Cu") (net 2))
 (arc (start 64.162499 65.361603) (mid 62.925 64.124103) (end 61.6875 65.361603) (width 2.138) (layer "F.Cu") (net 2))
 (arc (start 100.443499 88.9125) (mid 101.681 90.149999) (end 100.443499 91.3875) (width 2.138) (layer "F.Cu") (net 2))
 (arc (start 93.8625 64.0565) (mid 92.625 62.819) (end 91.3875 64.0565) (width 2.138) (layer "F.Cu") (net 2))
 (arc (start 71.587499 85.2) (mid 70.35 86.4375) (end 69.1125 85.2) (width 2.138) (layer "F.Cu") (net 2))
 (arc (start 74.0625 57.8065) (mid 72.825 56.568999) (end 71.587499 57.8065) (width 2.138) (layer "F.Cu") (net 2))
 (arc (start 81.4875 85.2) (mid 80.25 86.4375) (end 79.0125 85.2) (width 2.138) (layer "F.Cu") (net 2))
 (arc (start 83.962499 57.8065) (mid 82.725 56.568999) (end 81.4875 57.8065) (width 2.138) (layer "F.Cu") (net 2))
 (arc (start 97.574999 56.568999) (mid 100.200133 57.656366) (end 101.2875 60.281499) (width 2.138) (layer "F.Cu") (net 2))
 (arc (start 57.8065 96.337499) (mid 56.568999 97.574999) (end 57.8065 98.8125) (width 2.138) (layer "F.Cu") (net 2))
 (arc (start 79.0125 57.8065) (mid 77.774999 56.568999) (end 76.5375 57.8065) (width 2.138) (layer "F.Cu") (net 2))
 (arc (start 57.8065 101.2875) (mid 56.568999 102.524999) (end 57.8065 103.762499) (width 2.138) (layer "F.Cu") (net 2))
 (arc (start 88.9125 57.8065) (mid 87.675 56.568999) (end 86.4375 57.8065) (width 2.138) (layer "F.Cu") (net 2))
 (arc (start 69.1125 57.8065) (mid 67.874999 56.568999) (end 66.6375 57.8065) (width 2.138) (layer "F.Cu") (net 2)))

